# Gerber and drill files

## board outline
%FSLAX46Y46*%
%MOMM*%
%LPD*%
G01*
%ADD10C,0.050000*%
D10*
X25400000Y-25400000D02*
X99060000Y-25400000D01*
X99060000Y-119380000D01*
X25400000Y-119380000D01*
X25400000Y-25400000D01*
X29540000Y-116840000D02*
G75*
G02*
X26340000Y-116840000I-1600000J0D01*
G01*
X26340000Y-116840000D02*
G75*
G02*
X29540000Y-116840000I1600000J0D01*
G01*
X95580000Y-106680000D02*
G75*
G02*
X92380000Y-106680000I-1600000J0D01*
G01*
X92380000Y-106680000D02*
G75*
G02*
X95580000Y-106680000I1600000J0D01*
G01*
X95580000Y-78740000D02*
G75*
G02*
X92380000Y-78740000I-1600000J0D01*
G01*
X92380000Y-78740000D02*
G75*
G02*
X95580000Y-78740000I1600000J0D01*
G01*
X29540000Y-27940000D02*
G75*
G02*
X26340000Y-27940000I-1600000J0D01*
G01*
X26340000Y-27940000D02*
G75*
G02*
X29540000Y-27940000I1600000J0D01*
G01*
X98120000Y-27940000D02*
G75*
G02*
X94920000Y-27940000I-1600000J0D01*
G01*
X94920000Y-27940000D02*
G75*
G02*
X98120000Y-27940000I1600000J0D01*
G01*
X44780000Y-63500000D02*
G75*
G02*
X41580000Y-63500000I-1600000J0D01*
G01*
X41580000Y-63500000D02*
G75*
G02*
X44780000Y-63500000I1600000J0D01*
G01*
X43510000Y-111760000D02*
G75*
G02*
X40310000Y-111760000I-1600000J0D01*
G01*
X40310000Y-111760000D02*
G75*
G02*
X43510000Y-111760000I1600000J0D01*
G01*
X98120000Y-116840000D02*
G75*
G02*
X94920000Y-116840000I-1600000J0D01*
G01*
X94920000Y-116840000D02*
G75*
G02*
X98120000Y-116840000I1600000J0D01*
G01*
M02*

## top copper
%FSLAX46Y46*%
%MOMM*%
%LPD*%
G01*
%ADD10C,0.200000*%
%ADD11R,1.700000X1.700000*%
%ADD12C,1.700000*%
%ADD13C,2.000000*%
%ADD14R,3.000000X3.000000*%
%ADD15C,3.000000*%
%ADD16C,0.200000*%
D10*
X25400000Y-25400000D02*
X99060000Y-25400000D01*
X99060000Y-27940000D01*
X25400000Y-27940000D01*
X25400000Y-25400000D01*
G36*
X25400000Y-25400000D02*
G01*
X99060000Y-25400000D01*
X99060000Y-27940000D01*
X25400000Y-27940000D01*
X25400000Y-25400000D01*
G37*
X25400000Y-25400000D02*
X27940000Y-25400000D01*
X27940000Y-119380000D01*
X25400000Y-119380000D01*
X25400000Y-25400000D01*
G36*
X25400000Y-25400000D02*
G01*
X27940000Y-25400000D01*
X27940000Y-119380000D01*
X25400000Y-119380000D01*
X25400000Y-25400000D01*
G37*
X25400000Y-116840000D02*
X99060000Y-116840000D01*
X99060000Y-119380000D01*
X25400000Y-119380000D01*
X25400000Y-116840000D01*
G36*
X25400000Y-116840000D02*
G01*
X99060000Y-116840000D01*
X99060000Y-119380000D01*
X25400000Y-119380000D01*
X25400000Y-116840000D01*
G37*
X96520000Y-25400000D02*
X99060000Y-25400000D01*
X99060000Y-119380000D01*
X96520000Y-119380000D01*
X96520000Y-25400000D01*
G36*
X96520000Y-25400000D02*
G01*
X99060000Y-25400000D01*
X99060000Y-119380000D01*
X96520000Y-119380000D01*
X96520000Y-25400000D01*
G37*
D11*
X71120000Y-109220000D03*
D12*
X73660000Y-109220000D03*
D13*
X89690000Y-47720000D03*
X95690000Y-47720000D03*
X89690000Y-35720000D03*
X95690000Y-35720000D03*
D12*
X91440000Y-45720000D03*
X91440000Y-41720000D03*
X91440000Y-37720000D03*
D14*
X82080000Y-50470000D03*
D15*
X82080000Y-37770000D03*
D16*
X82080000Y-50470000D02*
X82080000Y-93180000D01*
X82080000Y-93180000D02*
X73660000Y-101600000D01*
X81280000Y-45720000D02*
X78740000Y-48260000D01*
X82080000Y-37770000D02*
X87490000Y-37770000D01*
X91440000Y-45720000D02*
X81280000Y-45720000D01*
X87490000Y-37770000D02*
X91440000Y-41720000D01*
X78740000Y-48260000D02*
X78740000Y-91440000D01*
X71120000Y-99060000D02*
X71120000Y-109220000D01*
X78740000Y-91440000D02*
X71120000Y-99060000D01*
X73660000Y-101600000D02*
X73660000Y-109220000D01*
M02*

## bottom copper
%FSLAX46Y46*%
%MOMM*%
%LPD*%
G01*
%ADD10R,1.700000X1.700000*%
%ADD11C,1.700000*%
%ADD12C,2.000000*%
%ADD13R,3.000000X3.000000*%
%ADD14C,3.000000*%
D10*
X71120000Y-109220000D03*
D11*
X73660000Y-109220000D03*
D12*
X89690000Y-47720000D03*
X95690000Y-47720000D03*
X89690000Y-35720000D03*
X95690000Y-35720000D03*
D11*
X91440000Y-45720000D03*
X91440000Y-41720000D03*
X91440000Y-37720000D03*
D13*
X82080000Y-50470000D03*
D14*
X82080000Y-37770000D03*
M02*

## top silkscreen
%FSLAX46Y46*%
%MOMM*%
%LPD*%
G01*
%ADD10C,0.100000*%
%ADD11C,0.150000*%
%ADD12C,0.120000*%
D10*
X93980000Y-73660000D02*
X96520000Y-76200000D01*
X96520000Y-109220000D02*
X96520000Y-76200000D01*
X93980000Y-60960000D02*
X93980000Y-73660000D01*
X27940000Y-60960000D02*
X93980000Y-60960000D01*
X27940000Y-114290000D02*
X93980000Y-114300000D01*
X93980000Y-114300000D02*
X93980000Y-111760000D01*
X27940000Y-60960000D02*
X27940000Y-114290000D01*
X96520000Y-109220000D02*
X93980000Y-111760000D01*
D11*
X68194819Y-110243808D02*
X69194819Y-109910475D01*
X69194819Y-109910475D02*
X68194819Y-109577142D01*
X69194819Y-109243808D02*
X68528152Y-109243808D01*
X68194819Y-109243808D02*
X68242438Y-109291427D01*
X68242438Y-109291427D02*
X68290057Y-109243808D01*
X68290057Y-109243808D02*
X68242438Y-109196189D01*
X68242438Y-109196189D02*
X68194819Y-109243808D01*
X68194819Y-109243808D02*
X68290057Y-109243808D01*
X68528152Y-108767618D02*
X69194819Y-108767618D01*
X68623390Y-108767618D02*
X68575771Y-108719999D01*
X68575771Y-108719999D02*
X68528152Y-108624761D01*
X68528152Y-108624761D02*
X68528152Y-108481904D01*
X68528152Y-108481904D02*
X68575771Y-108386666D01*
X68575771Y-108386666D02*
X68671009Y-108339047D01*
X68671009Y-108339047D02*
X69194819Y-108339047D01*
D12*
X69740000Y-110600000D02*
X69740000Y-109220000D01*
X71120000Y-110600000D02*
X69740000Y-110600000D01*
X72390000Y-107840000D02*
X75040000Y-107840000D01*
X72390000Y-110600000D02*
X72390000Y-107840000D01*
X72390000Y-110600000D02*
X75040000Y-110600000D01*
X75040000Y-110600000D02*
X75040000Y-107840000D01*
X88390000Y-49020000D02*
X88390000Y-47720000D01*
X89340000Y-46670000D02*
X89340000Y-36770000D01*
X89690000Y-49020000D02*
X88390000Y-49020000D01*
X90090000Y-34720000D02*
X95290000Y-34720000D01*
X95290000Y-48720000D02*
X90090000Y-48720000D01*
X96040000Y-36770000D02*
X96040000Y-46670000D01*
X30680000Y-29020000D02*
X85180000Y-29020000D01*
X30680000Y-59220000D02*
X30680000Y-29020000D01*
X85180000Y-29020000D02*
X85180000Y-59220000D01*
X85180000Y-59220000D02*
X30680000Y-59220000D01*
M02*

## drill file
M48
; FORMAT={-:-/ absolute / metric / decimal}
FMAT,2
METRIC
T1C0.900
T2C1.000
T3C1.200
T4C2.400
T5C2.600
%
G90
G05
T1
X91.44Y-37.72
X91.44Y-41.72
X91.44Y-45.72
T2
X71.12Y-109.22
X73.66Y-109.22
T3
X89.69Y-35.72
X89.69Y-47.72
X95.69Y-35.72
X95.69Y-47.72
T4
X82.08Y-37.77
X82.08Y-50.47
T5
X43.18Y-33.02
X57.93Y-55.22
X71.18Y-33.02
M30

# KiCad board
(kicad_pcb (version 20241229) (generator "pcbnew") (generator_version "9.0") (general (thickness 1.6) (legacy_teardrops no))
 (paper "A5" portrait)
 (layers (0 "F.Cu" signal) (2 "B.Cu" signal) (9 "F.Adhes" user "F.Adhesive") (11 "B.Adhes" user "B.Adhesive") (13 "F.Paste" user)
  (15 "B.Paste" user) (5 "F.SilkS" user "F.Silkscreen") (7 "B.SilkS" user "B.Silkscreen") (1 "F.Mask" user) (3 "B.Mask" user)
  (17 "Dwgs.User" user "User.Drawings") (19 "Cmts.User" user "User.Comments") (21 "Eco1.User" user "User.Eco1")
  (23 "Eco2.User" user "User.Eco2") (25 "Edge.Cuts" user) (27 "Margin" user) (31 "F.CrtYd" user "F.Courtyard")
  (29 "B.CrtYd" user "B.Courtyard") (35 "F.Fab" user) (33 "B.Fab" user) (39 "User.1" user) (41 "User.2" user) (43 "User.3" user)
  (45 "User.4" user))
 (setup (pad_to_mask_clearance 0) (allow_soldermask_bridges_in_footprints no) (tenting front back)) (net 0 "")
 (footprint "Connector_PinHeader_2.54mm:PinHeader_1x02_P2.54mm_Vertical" (layer "F.Cu") (at 71.12 109.22 90)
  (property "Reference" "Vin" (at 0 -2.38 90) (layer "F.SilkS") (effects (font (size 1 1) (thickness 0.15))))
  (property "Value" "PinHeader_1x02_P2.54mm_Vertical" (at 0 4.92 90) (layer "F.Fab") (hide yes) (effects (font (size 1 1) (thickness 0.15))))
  (fp_line (start -1.38 -1.38) (end 0 -1.38) (stroke (width 0.12) (type solid)) (layer "F.SilkS"))
  (fp_line (start -1.38 0) (end -1.38 -1.38) (stroke (width 0.12) (type solid)) (layer "F.SilkS"))
  (fp_line (start 1.38 1.27) (end 1.38 3.92) (stroke (width 0.12) (type solid)) (layer "F.SilkS"))
  (fp_line (start -1.38 1.27) (end 1.38 1.27) (stroke (width 0.12) (type solid)) (layer "F.SilkS"))
  (fp_line (start -1.38 1.27) (end -1.38 3.92) (stroke (width 0.12) (type solid)) (layer "F.SilkS"))
  (fp_line (start -1.38 3.92) (end 1.38 3.92) (stroke (width 0.12) (type solid)) (layer "F.SilkS"))
  (pad "1" thru_hole rect (at 0 0 90) (size 1.7 1.7) (drill 1) (layers "*.Cu" "*.Mask") (remove_unused_layers no))
  (pad "2" thru_hole circle (at 0 2.54 90) (size 1.7 1.7) (drill 1) (layers "*.Cu" "*.Mask") (remove_unused_layers no)))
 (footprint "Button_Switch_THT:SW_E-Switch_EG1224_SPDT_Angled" (layer "F.Cu") (at 91.44 45.72 90)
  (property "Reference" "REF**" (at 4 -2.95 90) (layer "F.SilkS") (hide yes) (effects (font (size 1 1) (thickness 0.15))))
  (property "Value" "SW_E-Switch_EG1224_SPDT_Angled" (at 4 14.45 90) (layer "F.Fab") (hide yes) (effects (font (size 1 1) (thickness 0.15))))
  (fp_line (start -3.3 -3.05) (end -2 -3.05) (stroke (width 0.12) (type solid)) (layer "F.SilkS"))
  (fp_line (start -0.95 -2.1) (end 8.95 -2.1) (stroke (width 0.12) (type solid)) (layer "F.SilkS"))
  (fp_line (start -3.3 -1.75) (end -3.3 -3.05) (stroke (width 0.12) (type solid)) (layer "F.SilkS"))
  (fp_line (start 11 -1.35) (end 11 3.85) (stroke (width 0.12) (type solid)) (layer "F.SilkS"))
  (fp_line (start -3 3.85) (end -3 -1.35) (stroke (width 0.12) (type solid)) (layer "F.SilkS"))
  (fp_line (start 8.95 4.6) (end -0.95 4.6) (stroke (width 0.12) (type solid)) (layer "F.SilkS"))
  (pad "" thru_hole circle (at -2 -1.75 90) (size 2 2) (drill 1.2) (layers "*.Cu" "*.Mask") (remove_unused_layers no))
  (pad "" thru_hole circle (at -2 4.25 90) (size 2 2) (drill 1.2) (layers "*.Cu" "*.Mask") (remove_unused_layers no))
  (pad "" thru_hole circle (at 10 -1.75 90) (size 2 2) (drill 1.2) (layers "*.Cu" "*.Mask") (remove_unused_layers no))
  (pad "" thru_hole circle (at 10 4.25 90) (size 2 2) (drill 1.2) (layers "*.Cu" "*.Mask") (remove_unused_layers no))
  (pad "1" thru_hole circle (at 0 0 90) (size 1.7 1.7) (drill 0.9) (layers "*.Cu" "*.Mask") (remove_unused_layers no))
  (pad "2" thru_hole circle (at 4 0 90) (size 1.7 1.7) (drill 0.9) (layers "*.Cu" "*.Mask") (remove_unused_layers no))
  (pad "3" thru_hole circle (at 8 0 90) (size 1.7 1.7) (drill 0.9) (layers "*.Cu" "*.Mask") (remove_unused_layers no)))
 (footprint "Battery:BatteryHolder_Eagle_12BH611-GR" (layer "F.Cu") (at 82.08 50.47)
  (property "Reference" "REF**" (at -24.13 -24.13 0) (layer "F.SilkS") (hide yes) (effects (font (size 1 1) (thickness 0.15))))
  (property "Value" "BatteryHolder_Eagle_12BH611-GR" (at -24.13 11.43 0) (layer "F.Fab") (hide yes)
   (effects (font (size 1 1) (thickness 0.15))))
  (fp_line (start -51.4 -21.45) (end 3.1 -21.45) (stroke (width 0.12) (type solid)) (layer "F.SilkS"))
  (fp_line (start -51.4 8.75) (end -51.4 -21.45) (stroke (width 0.12) (type solid)) (layer "F.SilkS"))
  (fp_line (start 3.1 -21.45) (end 3.1 8.75) (stroke (width 0.12) (type solid)) (layer "F.SilkS"))
  (fp_line (start 3.1 8.75) (end -51.4 8.75) (stroke (width 0.12) (type solid)) (layer "F.SilkS"))
  (pad "" np_thru_hole circle (at -38.9 -17.45) (size 2.6 2.6) (drill 2.6) (layers "*.Cu" "*.Mask"))
  (pad "" np_thru_hole circle (at -24.15 4.75) (size 2.6 2.6) (drill 2.6) (layers "*.Cu" "*.Mask"))
  (pad "" np_thru_hole circle (at -10.9 -17.45) (size 2.6 2.6) (drill 2.6) (layers "*.Cu" "*.Mask"))
  (pad "1" thru_hole rect (at 0 0) (size 3 3) (drill 2.4) (layers "*.Cu" "*.Mask") (remove_unused_layers no))
  (pad "2" thru_hole circle (at 0 -12.7) (size 3 3) (drill 2.4) (layers "*.Cu" "*.Mask") (remove_unused_layers no)))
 (gr_rect (start 25.4 25.4) (end 99.06 27.94) (stroke (width 0.2) (type solid)) (fill yes) (layer "F.Cu"))
 (gr_rect (start 25.4 25.4) (end 27.94 119.38) (stroke (width 0.2) (type solid)) (fill yes) (layer "F.Cu"))
 (gr_rect (start 25.4 116.84) (end 99.06 119.38) (stroke (width 0.2) (type solid)) (fill yes) (layer "F.Cu"))
 (gr_rect (start 96.52 25.4) (end 99.06 119.38) (stroke (width 0.2) (type solid)) (fill yes) (layer "F.Cu"))
 (gr_line (start 93.98 73.66) (end 96.52 76.2) (stroke (width 0.1) (type solid)) (layer "F.SilkS"))
 (gr_line (start 96.52 109.22) (end 96.52 76.2) (stroke (width 0.1) (type solid)) (layer "F.SilkS"))
 (gr_line (start 93.98 60.96) (end 93.98 73.66) (stroke (width 0.1) (type solid)) (layer "F.SilkS"))
 (gr_line (start 27.94 60.96) (end 93.98 60.96) (stroke (width 0.1) (type solid)) (layer "F.SilkS"))
 (gr_line (start 27.94 114.29) (end 93.98 114.3) (stroke (width 0.1) (type solid)) (layer "F.SilkS"))
 (gr_line (start 93.98 114.3) (end 93.98 111.76) (stroke (width 0.1) (type solid)) (layer "F.SilkS"))
 (gr_line (start 27.94 60.96) (end 27.94 114.29) (stroke (width 0.1) (type solid)) (layer "F.SilkS"))
 (gr_line (start 96.52 109.22) (end 93.98 111.76) (stroke (width 0.1) (type default)) (layer "F.SilkS"))
 (gr_rect (start 25.4 25.4) (end 99.06 119.38) (stroke (width 0.05) (type default)) (fill no) (layer "Edge.Cuts"))
 (gr_circle (center 27.94 116.84) (end 29.54 116.84) (stroke (width 0.05) (type solid)) (fill no) (layer "Edge.Cuts"))
 (gr_circle (center 93.98 106.68) (end 95.58 106.68) (stroke (width 0.05) (type solid)) (fill no) (layer "Edge.Cuts"))
 (gr_circle (center 93.98 78.74) (end 95.58 78.74) (stroke (width 0.05) (type solid)) (fill no) (layer "Edge.Cuts"))
 (gr_circle (center 27.94 27.94) (end 29.54 27.94) (stroke (width 0.05) (type solid)) (fill no) (layer "Edge.Cuts"))
 (gr_circle (center 96.52 27.94) (end 98.12 27.94) (stroke (width 0.05) (type solid)) (fill no) (layer "Edge.Cuts"))
 (gr_circle (center 43.18 63.5) (end 44.78 63.5) (stroke (width 0.05) (type solid)) (fill no) (layer "Edge.Cuts"))
 (gr_circle (center 41.91 111.76) (end 43.51 111.76) (stroke (width 0.05) (type solid)) (fill no) (layer "Edge.Cuts"))
 (gr_circle (center 96.52 116.84) (end 98.12 116.84) (stroke (width 0.05) (type solid)) (fill no) (layer "Edge.Cuts"))
 (segment (start 82.08 50.47) (end 82.08 93.18) (width 0.2) (layer "F.Cu") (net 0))
 (segment (start 82.08 93.18) (end 73.66 101.6) (width 0.2) (layer "F.Cu") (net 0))
 (segment (start 81.28 45.72) (end 78.74 48.26) (width 0.2) (layer "F.Cu") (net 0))
 (segment (start 82.08 37.77) (end 87.49 37.77) (width 0.2) (layer "F.Cu") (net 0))
 (segment (start 91.44 45.72) (end 81.28 45.72) (width 0.2) (layer "F.Cu") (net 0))
 (segment (start 87.49 37.77) (end 91.44 41.72) (width 0.2) (layer "F.Cu") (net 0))
 (segment (start 78.74 48.26) (end 78.74 91.44) (width 0.2) (layer "F.Cu") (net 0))
 (segment (start 71.12 99.06) (end 71.12 109.22) (width 0.2) (layer "F.Cu") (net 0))
 (segment (start 78.74 91.44) (end 71.12 99.06) (width 0.2) (layer "F.Cu") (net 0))
 (segment (start 73.66 101.6) (end 73.66 109.22) (width 0.2) (layer "F.Cu") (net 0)))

